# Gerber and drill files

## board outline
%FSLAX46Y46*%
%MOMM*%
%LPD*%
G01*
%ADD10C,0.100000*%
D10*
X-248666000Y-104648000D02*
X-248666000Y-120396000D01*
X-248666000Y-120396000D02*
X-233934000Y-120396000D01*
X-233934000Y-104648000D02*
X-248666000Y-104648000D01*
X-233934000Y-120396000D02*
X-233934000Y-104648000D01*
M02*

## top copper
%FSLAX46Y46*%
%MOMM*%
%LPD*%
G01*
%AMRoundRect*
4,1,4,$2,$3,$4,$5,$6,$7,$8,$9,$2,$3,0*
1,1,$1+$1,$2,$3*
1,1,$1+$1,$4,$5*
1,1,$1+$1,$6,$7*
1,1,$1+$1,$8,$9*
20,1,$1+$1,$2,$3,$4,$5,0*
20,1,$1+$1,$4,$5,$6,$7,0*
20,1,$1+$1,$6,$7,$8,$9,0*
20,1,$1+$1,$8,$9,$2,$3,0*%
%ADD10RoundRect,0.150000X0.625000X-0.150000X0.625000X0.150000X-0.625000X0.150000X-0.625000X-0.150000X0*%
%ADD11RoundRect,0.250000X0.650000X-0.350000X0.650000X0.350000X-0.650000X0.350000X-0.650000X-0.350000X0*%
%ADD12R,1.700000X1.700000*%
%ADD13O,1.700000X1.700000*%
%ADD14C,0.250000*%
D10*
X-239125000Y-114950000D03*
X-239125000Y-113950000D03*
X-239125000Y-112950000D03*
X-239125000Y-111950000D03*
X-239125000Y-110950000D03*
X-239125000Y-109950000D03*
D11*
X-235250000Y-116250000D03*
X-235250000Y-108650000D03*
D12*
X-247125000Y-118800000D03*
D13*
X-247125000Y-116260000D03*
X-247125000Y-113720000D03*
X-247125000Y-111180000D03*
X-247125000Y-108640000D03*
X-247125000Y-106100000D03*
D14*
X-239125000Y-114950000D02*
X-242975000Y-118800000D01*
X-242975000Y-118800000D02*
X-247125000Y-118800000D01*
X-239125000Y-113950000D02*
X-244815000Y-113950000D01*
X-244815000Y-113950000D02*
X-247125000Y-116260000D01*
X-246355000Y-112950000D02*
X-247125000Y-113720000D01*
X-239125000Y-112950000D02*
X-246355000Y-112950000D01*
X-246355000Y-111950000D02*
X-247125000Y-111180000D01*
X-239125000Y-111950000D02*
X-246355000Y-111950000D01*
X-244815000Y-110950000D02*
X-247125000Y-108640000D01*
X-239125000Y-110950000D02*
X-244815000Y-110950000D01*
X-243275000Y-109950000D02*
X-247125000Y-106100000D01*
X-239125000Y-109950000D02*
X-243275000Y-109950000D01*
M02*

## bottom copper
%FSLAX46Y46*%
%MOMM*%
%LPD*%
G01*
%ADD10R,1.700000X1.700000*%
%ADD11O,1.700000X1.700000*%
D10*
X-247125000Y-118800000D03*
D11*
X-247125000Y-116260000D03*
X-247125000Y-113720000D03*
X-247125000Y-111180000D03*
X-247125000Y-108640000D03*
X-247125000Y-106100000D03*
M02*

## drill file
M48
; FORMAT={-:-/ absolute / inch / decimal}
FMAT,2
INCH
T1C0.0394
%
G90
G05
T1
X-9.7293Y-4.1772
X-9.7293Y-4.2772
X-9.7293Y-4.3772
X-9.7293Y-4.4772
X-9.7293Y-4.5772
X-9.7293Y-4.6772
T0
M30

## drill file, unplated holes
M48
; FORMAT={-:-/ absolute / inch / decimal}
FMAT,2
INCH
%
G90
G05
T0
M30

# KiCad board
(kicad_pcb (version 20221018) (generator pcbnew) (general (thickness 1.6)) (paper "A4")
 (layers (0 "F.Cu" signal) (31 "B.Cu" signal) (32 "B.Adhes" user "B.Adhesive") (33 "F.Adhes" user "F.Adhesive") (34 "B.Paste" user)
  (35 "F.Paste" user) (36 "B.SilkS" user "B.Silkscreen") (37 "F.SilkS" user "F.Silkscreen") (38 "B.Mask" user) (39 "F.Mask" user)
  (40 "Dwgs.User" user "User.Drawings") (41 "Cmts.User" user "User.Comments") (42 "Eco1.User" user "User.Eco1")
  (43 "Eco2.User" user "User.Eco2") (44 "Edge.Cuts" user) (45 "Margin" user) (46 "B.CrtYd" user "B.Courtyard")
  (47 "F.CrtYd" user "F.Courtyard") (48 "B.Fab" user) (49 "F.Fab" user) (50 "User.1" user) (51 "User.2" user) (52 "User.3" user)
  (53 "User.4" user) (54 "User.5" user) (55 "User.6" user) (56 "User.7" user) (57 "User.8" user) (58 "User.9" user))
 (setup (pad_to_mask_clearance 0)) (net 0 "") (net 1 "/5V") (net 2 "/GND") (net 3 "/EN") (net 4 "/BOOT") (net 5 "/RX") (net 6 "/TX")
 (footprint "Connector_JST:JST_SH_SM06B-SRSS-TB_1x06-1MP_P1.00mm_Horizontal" (layer "F.Cu") (at -237.125 112.45 90)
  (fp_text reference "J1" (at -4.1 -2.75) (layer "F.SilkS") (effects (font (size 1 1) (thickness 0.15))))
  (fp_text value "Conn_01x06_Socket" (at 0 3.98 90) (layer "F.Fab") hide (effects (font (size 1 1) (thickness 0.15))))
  (pad "1" smd roundrect (at -2.5 -2 90) (size 0.6 1.55) (layers "F.Cu" "F.Paste" "F.Mask") (roundrect_rratio 0.25) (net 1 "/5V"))
  (pad "2" smd roundrect (at -1.5 -2 90) (size 0.6 1.55) (layers "F.Cu" "F.Paste" "F.Mask") (roundrect_rratio 0.25) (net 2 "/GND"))
  (pad "3" smd roundrect (at -0.5 -2 90) (size 0.6 1.55) (layers "F.Cu" "F.Paste" "F.Mask") (roundrect_rratio 0.25) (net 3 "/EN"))
  (pad "4" smd roundrect (at 0.5 -2 90) (size 0.6 1.55) (layers "F.Cu" "F.Paste" "F.Mask") (roundrect_rratio 0.25) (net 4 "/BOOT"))
  (pad "5" smd roundrect (at 1.5 -2 90) (size 0.6 1.55) (layers "F.Cu" "F.Paste" "F.Mask") (roundrect_rratio 0.25) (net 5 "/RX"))
  (pad "6" smd roundrect (at 2.5 -2 90) (size 0.6 1.55) (layers "F.Cu" "F.Paste" "F.Mask") (roundrect_rratio 0.25) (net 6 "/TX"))
  (pad "MP" smd roundrect (at -3.8 1.875 90) (size 1.2 1.8) (layers "F.Cu" "F.Paste" "F.Mask") (roundrect_rratio 0.2083333333))
  (pad "MP" smd roundrect (at 3.8 1.875 90) (size 1.2 1.8) (layers "F.Cu" "F.Paste" "F.Mask") (roundrect_rratio 0.2083333333)))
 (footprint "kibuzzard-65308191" (layer "F.Cu") (at -237.236 106.172)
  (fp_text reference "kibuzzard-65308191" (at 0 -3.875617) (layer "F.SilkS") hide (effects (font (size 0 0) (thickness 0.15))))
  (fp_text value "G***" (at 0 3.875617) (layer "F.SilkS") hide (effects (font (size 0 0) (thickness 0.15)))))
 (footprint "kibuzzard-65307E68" (layer "F.Cu") (at -242.875 112.05)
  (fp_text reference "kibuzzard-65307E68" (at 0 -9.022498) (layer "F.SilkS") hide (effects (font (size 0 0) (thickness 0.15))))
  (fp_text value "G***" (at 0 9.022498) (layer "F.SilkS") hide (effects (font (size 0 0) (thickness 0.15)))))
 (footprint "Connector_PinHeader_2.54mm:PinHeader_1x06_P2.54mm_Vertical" (layer "B.Cu") (at -247.125 118.8)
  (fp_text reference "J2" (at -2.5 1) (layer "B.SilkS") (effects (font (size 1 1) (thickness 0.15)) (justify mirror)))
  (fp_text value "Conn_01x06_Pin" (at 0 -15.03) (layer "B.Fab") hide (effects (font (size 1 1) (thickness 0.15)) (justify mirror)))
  (pad "1" thru_hole rect (at 0 0) (size 1.7 1.7) (drill 1) (layers "*.Cu" "*.Mask") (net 1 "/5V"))
  (pad "2" thru_hole oval (at 0 -2.54) (size 1.7 1.7) (drill 1) (layers "*.Cu" "*.Mask") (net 2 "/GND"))
  (pad "3" thru_hole oval (at 0 -5.08) (size 1.7 1.7) (drill 1) (layers "*.Cu" "*.Mask") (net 3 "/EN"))
  (pad "4" thru_hole oval (at 0 -7.62) (size 1.7 1.7) (drill 1) (layers "*.Cu" "*.Mask") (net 4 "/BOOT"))
  (pad "5" thru_hole oval (at 0 -10.16) (size 1.7 1.7) (drill 1) (layers "*.Cu" "*.Mask") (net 5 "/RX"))
  (pad "6" thru_hole oval (at 0 -12.7) (size 1.7 1.7) (drill 1) (layers "*.Cu" "*.Mask") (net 6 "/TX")))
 (gr_line (start -248.666 104.648) (end -248.666 120.396) (stroke (width 0.1) (type default)) (layer "Edge.Cuts"))
 (gr_line (start -248.666 120.396) (end -233.934 120.396) (stroke (width 0.1) (type default)) (layer "Edge.Cuts"))
 (gr_line (start -233.934 104.648) (end -248.666 104.648) (stroke (width 0.1) (type default)) (layer "Edge.Cuts"))
 (gr_line (start -233.934 120.396) (end -233.934 104.648) (stroke (width 0.1) (type default)) (layer "Edge.Cuts"))
 (segment (start -239.125 114.95) (end -242.975 118.8) (width 0.25) (layer "F.Cu") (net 1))
 (segment (start -242.975 118.8) (end -247.125 118.8) (width 0.25) (layer "F.Cu") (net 1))
 (segment (start -239.125 113.95) (end -244.815 113.95) (width 0.25) (layer "F.Cu") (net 2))
 (segment (start -244.815 113.95) (end -247.125 116.26) (width 0.25) (layer "F.Cu") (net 2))
 (segment (start -246.355 112.95) (end -247.125 113.72) (width 0.25) (layer "F.Cu") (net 3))
 (segment (start -239.125 112.95) (end -246.355 112.95) (width 0.25) (layer "F.Cu") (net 3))
 (segment (start -246.355 111.95) (end -247.125 111.18) (width 0.25) (layer "F.Cu") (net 4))
 (segment (start -239.125 111.95) (end -246.355 111.95) (width 0.25) (layer "F.Cu") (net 4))
 (segment (start -244.815 110.95) (end -247.125 108.64) (width 0.25) (layer "F.Cu") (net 5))
 (segment (start -239.125 110.95) (end -244.815 110.95) (width 0.25) (layer "F.Cu") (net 5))
 (segment (start -243.275 109.95) (end -247.125 106.1) (width 0.25) (layer "F.Cu") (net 6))
 (segment (start -239.125 109.95) (end -243.275 109.95) (width 0.25) (layer "F.Cu") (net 6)))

